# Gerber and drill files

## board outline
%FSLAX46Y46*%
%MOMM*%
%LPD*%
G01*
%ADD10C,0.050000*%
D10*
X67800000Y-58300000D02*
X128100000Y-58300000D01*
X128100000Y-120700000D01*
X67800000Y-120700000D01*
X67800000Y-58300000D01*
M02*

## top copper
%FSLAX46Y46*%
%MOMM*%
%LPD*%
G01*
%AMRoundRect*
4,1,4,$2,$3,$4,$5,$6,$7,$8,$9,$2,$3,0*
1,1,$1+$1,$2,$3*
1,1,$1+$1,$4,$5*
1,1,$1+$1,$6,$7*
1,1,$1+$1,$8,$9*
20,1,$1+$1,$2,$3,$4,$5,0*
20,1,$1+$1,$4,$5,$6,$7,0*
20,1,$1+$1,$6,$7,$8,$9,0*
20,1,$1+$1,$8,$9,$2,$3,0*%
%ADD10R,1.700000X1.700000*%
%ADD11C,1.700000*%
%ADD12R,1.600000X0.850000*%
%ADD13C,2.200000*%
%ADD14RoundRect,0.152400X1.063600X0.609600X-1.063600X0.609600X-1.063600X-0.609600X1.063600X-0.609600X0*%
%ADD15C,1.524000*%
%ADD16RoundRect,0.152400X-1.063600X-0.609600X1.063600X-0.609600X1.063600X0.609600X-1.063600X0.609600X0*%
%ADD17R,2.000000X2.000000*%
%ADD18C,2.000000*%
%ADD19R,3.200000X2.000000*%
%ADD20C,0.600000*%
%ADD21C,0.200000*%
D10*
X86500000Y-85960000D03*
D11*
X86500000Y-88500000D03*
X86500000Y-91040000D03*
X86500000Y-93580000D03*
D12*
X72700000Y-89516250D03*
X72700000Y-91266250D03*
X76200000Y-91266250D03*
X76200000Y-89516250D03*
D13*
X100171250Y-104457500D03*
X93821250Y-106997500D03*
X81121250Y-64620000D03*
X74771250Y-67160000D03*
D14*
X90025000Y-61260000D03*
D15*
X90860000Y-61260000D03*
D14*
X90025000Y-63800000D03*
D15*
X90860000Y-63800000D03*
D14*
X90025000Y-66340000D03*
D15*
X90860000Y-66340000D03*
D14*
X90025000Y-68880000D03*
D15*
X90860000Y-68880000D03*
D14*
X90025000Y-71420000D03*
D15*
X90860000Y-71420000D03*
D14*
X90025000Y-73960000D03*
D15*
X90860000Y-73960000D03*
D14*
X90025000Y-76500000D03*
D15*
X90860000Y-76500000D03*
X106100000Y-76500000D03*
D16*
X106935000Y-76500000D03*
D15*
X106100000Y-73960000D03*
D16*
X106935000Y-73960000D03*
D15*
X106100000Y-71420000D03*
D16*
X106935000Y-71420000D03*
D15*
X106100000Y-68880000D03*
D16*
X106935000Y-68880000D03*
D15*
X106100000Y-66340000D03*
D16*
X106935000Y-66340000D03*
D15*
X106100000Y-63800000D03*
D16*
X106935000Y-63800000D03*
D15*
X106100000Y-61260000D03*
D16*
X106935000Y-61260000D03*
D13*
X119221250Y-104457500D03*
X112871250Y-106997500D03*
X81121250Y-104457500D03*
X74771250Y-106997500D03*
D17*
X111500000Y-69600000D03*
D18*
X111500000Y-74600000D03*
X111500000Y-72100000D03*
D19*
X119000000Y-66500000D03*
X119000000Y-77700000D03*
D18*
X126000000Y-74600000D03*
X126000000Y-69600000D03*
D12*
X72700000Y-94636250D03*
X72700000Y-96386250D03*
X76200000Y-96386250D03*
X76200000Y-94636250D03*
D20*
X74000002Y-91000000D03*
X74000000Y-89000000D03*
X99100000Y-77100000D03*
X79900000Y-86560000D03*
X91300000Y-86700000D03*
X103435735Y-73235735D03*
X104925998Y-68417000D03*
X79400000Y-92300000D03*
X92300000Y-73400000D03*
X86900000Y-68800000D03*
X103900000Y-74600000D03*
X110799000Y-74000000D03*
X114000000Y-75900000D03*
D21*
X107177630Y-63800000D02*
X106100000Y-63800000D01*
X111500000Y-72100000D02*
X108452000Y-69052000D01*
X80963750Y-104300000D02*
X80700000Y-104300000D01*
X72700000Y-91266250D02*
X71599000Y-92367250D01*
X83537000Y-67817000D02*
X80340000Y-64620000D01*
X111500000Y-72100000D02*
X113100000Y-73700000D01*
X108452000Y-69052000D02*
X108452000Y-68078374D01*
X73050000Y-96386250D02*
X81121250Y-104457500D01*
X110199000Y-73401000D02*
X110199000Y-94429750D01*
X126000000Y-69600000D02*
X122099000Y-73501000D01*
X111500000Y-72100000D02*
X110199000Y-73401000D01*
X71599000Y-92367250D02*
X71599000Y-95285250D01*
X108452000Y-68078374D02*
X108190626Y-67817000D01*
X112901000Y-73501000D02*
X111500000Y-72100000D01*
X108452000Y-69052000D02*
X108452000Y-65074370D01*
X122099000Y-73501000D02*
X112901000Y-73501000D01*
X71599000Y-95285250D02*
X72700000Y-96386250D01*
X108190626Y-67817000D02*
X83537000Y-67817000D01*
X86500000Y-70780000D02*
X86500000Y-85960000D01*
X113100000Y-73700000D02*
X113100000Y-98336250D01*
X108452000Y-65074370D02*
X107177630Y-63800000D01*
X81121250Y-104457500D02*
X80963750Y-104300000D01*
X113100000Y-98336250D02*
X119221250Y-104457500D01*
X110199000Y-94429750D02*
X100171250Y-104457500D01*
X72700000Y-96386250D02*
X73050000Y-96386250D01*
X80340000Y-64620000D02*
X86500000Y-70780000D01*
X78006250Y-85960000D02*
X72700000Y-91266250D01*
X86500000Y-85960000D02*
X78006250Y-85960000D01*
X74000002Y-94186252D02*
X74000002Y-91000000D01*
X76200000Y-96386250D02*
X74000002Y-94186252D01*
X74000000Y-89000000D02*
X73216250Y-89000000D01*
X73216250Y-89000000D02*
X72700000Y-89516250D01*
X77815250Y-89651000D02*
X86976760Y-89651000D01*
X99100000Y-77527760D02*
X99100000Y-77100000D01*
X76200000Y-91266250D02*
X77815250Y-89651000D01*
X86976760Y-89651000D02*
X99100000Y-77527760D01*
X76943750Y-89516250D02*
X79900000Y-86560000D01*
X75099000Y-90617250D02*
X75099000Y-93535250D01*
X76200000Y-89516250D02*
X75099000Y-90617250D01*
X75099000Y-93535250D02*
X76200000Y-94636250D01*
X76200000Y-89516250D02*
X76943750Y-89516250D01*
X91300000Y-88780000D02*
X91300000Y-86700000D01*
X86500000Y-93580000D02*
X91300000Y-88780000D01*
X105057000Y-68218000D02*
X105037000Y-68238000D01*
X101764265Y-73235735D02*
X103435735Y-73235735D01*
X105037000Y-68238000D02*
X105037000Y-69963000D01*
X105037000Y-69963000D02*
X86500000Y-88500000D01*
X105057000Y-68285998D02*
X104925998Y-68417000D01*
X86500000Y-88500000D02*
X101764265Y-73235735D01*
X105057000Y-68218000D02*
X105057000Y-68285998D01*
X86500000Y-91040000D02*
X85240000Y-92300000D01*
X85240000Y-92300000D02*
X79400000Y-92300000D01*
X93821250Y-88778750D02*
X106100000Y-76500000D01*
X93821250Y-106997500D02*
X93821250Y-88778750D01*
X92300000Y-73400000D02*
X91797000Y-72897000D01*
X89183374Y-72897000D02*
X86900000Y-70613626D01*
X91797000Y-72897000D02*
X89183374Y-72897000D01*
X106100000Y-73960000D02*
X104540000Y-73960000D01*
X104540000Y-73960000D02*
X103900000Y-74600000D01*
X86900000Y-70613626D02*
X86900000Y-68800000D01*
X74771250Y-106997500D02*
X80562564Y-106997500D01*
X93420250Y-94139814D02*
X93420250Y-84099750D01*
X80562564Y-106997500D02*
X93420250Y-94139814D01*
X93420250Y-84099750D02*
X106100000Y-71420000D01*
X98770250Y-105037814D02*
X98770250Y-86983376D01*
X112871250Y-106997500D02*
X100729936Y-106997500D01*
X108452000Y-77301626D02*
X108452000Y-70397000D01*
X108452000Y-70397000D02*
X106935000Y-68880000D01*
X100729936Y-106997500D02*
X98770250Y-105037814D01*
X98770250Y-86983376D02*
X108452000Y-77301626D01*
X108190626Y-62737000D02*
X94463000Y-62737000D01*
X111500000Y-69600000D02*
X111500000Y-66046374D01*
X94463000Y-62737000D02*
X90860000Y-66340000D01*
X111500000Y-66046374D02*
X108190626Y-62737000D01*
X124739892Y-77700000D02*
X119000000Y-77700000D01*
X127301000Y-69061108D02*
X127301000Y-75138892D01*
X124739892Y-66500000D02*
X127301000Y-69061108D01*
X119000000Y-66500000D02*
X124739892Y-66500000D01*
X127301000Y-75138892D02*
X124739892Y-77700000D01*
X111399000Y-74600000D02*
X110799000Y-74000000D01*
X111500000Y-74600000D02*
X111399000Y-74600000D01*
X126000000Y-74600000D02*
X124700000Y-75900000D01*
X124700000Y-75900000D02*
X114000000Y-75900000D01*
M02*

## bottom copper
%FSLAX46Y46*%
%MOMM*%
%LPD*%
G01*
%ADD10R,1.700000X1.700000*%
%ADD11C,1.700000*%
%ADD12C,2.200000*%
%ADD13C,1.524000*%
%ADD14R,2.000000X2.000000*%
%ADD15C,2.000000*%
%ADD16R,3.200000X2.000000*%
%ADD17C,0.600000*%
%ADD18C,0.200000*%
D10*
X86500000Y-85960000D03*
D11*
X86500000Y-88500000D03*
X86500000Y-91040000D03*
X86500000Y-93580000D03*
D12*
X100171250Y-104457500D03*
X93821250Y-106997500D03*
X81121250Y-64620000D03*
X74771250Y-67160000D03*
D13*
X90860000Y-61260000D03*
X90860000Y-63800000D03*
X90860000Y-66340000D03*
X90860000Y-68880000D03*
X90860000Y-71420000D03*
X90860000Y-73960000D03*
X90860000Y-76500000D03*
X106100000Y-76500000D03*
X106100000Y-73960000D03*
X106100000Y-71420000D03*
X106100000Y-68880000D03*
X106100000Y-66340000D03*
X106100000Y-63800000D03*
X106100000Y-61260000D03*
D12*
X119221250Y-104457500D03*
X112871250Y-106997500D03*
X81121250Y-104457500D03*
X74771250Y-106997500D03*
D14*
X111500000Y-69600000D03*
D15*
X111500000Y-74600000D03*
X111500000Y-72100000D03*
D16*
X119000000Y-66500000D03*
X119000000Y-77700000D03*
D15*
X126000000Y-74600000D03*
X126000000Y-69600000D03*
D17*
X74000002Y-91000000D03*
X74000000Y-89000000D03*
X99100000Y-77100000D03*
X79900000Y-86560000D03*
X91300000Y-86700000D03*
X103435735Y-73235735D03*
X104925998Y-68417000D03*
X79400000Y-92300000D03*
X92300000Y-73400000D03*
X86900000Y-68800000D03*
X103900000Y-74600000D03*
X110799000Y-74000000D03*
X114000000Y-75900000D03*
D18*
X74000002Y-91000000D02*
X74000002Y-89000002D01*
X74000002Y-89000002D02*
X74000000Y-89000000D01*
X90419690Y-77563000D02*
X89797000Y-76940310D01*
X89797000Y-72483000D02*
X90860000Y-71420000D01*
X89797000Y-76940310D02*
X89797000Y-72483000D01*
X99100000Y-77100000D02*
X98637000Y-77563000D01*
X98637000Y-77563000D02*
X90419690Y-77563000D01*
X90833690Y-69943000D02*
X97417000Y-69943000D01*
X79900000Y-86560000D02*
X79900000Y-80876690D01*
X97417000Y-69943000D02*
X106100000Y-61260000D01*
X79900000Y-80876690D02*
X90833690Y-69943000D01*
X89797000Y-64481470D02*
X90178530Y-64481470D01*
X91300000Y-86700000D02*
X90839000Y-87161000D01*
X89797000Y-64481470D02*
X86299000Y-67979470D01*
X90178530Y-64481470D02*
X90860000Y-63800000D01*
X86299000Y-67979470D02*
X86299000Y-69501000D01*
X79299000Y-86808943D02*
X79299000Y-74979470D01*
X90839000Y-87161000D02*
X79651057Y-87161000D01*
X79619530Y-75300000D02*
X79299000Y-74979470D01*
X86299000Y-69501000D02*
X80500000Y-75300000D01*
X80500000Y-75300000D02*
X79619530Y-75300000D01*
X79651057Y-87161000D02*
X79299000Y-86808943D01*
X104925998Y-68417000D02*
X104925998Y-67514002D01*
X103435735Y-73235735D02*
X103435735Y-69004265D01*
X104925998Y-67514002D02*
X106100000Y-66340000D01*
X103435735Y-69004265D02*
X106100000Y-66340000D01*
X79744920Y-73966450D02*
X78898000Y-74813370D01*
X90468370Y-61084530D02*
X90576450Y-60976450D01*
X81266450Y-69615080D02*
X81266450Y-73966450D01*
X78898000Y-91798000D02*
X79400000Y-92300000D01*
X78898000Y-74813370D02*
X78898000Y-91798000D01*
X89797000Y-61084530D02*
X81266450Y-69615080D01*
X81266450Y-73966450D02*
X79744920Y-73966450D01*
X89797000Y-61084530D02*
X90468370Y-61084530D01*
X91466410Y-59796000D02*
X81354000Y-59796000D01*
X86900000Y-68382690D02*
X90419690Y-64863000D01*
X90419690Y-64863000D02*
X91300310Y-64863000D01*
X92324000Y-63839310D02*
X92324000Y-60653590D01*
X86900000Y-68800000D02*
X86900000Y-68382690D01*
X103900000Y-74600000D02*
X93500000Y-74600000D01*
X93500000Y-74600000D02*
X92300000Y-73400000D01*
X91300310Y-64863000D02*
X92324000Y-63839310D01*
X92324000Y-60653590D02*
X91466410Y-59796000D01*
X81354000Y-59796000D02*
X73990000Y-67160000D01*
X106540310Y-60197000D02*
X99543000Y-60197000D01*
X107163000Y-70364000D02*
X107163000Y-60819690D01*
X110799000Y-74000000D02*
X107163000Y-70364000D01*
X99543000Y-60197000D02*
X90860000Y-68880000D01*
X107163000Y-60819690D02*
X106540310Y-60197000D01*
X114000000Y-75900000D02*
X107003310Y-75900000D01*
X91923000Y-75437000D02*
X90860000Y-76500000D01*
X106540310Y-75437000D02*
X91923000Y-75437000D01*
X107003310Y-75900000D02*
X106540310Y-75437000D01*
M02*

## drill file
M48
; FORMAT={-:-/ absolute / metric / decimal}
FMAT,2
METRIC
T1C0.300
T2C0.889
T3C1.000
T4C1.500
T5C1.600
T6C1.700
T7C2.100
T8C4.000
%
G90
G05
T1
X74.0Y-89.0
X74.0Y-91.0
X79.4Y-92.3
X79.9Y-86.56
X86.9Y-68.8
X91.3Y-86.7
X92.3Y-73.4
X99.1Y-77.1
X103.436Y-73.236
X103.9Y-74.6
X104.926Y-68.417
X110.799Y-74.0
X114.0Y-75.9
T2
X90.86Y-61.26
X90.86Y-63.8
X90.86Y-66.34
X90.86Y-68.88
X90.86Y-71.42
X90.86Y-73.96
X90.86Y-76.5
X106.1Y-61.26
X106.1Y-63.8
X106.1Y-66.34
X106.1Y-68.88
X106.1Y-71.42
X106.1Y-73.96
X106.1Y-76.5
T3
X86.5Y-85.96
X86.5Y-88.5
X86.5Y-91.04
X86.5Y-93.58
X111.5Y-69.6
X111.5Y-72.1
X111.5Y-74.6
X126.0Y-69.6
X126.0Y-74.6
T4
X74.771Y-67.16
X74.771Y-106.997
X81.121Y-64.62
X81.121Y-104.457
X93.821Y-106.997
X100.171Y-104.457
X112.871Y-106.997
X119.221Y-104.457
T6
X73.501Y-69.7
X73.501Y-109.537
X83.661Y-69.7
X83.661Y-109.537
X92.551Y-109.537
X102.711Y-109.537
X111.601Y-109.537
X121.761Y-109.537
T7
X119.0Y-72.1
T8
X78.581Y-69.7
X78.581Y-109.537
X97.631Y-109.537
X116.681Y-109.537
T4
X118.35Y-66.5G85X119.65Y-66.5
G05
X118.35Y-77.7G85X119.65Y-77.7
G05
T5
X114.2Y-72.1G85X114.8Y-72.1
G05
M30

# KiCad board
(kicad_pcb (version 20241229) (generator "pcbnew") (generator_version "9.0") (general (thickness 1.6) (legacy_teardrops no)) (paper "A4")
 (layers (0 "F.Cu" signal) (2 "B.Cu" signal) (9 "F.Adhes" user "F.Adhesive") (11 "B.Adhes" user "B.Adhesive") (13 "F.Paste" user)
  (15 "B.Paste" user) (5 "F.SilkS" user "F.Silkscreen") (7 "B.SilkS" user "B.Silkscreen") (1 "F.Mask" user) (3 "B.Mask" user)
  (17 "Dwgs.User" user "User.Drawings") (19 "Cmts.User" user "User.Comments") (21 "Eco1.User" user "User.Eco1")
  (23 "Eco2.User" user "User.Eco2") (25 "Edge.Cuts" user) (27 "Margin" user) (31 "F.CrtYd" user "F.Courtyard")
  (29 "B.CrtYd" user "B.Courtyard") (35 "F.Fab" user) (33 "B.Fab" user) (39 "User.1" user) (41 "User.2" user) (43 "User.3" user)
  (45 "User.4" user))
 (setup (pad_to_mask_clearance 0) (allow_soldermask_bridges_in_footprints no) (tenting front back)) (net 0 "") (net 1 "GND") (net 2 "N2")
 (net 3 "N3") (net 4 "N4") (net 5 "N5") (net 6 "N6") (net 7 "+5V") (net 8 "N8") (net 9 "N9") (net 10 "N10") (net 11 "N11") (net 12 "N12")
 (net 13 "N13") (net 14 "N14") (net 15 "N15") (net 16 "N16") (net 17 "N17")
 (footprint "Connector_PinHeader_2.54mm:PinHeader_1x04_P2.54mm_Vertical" (layer "F.Cu") (at 86.5 85.96)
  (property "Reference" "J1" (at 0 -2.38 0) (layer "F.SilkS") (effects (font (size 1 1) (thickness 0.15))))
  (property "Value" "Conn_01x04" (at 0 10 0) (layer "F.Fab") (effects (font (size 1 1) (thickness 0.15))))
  (pad "1" thru_hole rect (at 0 0) (size 1.7 1.7) (drill 1) (layers "*.Cu" "*.Mask") (remove_unused_layers no) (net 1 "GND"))
  (pad "2" thru_hole circle (at 0 2.54) (size 1.7 1.7) (drill 1) (layers "*.Cu" "*.Mask") (remove_unused_layers no) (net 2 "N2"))
  (pad "3" thru_hole circle (at 0 5.08) (size 1.7 1.7) (drill 1) (layers "*.Cu" "*.Mask") (remove_unused_layers no) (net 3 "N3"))
  (pad "4" thru_hole circle (at 0 7.62) (size 1.7 1.7) (drill 1) (layers "*.Cu" "*.Mask") (remove_unused_layers no) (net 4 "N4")))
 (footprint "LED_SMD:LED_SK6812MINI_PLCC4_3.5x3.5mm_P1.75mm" (layer "F.Cu") (at 74.45 90.39125)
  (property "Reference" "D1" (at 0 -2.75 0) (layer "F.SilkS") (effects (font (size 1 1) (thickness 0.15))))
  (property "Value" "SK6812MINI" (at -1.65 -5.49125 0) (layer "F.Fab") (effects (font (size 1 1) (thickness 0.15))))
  (pad "1" smd rect (at -1.75 -0.875) (size 1.6 0.85) (layers "F.Cu" "F.Mask" "F.Paste") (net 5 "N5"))
  (pad "2" smd rect (at -1.75 0.875) (size 1.6 0.85) (layers "F.Cu" "F.Mask" "F.Paste") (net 1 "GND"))
  (pad "3" smd rect (at 1.75 0.875) (size 1.6 0.85) (layers "F.Cu" "F.Mask" "F.Paste") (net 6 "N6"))
  (pad "4" smd rect (at 1.75 -0.875) (size 1.6 0.85) (layers "F.Cu" "F.Mask" "F.Paste") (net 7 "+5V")))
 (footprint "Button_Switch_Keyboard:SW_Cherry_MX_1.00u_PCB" (layer "F.Cu") (at 100.17125 104.4575)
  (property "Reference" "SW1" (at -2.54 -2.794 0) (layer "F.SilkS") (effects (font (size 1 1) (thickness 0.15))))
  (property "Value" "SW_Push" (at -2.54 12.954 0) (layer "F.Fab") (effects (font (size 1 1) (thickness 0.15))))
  (pad "" np_thru_hole circle (at -7.62 5.08) (size 1.7 1.7) (drill 1.7) (layers "*.Cu" "*.Mask"))
  (pad "" np_thru_hole circle (at -2.54 5.08) (size 4 4) (drill 4) (layers "*.Cu" "*.Mask"))
  (pad "" np_thru_hole circle (at 2.54 5.08) (size 1.7 1.7) (drill 1.7) (layers "*.Cu" "*.Mask"))
  (pad "1" thru_hole circle (at 0 0) (size 2.2 2.2) (drill 1.5) (layers "*.Cu" "*.Mask") (remove_unused_layers no) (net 1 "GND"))
  (pad "2" thru_hole circle (at -6.35 2.54) (size 2.2 2.2) (drill 1.5) (layers "*.Cu" "*.Mask") (remove_unused_layers no) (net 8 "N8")))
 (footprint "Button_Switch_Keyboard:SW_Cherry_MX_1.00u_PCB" (layer "F.Cu") (at 81.12125 64.62)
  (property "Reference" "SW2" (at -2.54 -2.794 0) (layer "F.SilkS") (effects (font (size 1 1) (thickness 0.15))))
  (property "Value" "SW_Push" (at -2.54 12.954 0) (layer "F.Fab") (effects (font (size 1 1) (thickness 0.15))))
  (pad "" np_thru_hole circle (at -7.62 5.08) (size 1.7 1.7) (drill 1.7) (layers "*.Cu" "*.Mask"))
  (pad "" np_thru_hole circle (at -2.54 5.08) (size 4 4) (drill 4) (layers "*.Cu" "*.Mask"))
  (pad "" np_thru_hole circle (at 2.54 5.08) (size 1.7 1.7) (drill 1.7) (layers "*.Cu" "*.Mask"))
  (pad "1" thru_hole circle (at 0 0) (size 2.2 2.2) (drill 1.5) (layers "*.Cu" "*.Mask") (remove_unused_layers no) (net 1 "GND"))
  (pad "2" thru_hole circle (at -6.35 2.54) (size 2.2 2.2) (drill 1.5) (layers "*.Cu" "*.Mask") (remove_unused_layers no) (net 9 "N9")))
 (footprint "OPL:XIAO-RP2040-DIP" (layer "F.Cu") (at 98.48 68.88)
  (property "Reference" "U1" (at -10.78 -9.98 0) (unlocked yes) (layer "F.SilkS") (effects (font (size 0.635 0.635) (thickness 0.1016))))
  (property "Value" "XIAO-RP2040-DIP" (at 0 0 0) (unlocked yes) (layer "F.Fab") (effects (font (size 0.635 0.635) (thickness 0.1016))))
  (pad "1" smd roundrect (at -8.455 -7.62 180) (size 2.432 1.524) (layers "F.Cu" "F.Mask") (roundrect_rratio 0.1) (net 3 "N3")
   (thermal_bridge_angle 45))
  (pad "1" thru_hole circle (at -7.62 -7.62 180) (size 1.524 1.524) (drill 0.889) (layers "*.Cu" "*.Mask") (remove_unused_layers no)
   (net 3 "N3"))
  (pad "2" smd roundrect (at -8.455 -5.08 180) (size 2.432 1.524) (layers "F.Cu" "F.Mask") (roundrect_rratio 0.1) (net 4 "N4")
   (thermal_bridge_angle 45))
  (pad "2" thru_hole circle (at -7.62 -5.08 180) (size 1.524 1.524) (drill 0.889) (layers "*.Cu" "*.Mask") (remove_unused_layers no)
   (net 4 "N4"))
  (pad "3" smd roundrect (at -8.455 -2.54 180) (size 2.432 1.524) (layers "F.Cu" "F.Mask") (roundrect_rratio 0.1) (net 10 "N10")
   (thermal_bridge_angle 45))
  (pad "3" thru_hole circle (at -7.62 -2.54 180) (size 1.524 1.524) (drill 0.889) (layers "*.Cu" "*.Mask") (remove_unused_layers no)
   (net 10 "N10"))
  (pad "4" smd roundrect (at -8.455 0 180) (size 2.432 1.524) (layers "F.Cu" "F.Mask") (roundrect_rratio 0.1) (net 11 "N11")
   (thermal_bridge_angle 45))
  (pad "4" thru_hole circle (at -7.62 0 180) (size 1.524 1.524) (drill 0.889) (layers "*.Cu" "*.Mask") (remove_unused_layers no)
   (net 11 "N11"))
  (pad "5" smd roundrect (at -8.455 2.54 180) (size 2.432 1.524) (layers "F.Cu" "F.Mask") (roundrect_rratio 0.1) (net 6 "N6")
   (thermal_bridge_angle 45))
  (pad "5" thru_hole circle (at -7.62 2.54 180) (size 1.524 1.524) (drill 0.889) (layers "*.Cu" "*.Mask") (remove_unused_layers no)
   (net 6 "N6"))
  (pad "6" smd roundrect (at -8.455 5.08 180) (size 2.432 1.524) (layers "F.Cu" "F.Mask") (roundrect_rratio 0.1) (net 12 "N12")
   (thermal_bridge_angle 45))
  (pad "6" thru_hole circle (at -7.62 5.08 180) (size 1.524 1.524) (drill 0.889) (layers "*.Cu" "*.Mask") (remove_unused_layers no)
   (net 12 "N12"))
  (pad "7" smd roundrect (at -8.455 7.62 180) (size 2.432 1.524) (layers "F.Cu" "F.Mask") (roundrect_rratio 0.1) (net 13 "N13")
   (thermal_bridge_angle 45))
  (pad "7" thru_hole circle (at -7.62 7.62 180) (size 1.524 1.524) (drill 0.889) (layers "*.Cu" "*.Mask") (remove_unused_layers no)
   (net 13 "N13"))
  (pad "8" thru_hole circle (at 7.62 7.62) (size 1.524 1.524) (drill 0.889) (layers "*.Cu" "*.Mask") (remove_unused_layers no) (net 8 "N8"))
  (pad "8" smd roundrect (at 8.455 7.62) (size 2.432 1.524) (layers "F.Cu" "F.Mask") (roundrect_rratio 0.1) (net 8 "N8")
   (thermal_bridge_angle 45))
  (pad "9" thru_hole circle (at 7.62 5.08) (size 1.524 1.524) (drill 0.889) (layers "*.Cu" "*.Mask") (remove_unused_layers no) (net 9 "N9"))
  (pad "9" smd roundrect (at 8.455 5.08) (size 2.432 1.524) (layers "F.Cu" "F.Mask") (roundrect_rratio 0.1) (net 9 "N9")
   (thermal_bridge_angle 45))
  (pad "10" thru_hole circle (at 7.62 2.54) (size 1.524 1.524) (drill 0.889) (layers "*.Cu" "*.Mask") (remove_unused_layers no)
   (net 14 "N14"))
  (pad "10" smd roundrect (at 8.455 2.54) (size 2.432 1.524) (layers "F.Cu" "F.Mask") (roundrect_rratio 0.1) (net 14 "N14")
   (thermal_bridge_angle 45))
  (pad "11" thru_hole circle (at 7.62 0) (size 1.524 1.524) (drill 0.889) (layers "*.Cu" "*.Mask") (remove_unused_layers no) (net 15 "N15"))
  (pad "11" smd roundrect (at 8.455 0) (size 2.432 1.524) (layers "F.Cu" "F.Mask") (roundrect_rratio 0.1) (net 15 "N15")
   (thermal_bridge_angle 45))
  (pad "12" thru_hole circle (at 7.62 -2.54) (size 1.524 1.524) (drill 0.889) (layers "*.Cu" "*.Mask") (remove_unused_layers no)
   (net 2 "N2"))
  (pad "12" smd roundrect (at 8.455 -2.54) (size 2.432 1.524) (layers "F.Cu" "F.Mask") (roundrect_rratio 0.1) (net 2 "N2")
   (thermal_bridge_angle 45))
  (pad "13" thru_hole circle (at 7.62 -5.08) (size 1.524 1.524) (drill 0.889) (layers "*.Cu" "*.Mask") (remove_unused_layers no)
   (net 1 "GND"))
  (pad "13" smd roundrect (at 8.455 -5.08) (size 2.432 1.524) (layers "F.Cu" "F.Mask") (roundrect_rratio 0.1) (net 1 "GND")
   (thermal_bridge_angle 45))
  (pad "14" thru_hole circle (at 7.62 -7.62) (size 1.524 1.524) (drill 0.889) (layers "*.Cu" "*.Mask") (remove_unused_layers no)
   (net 7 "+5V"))
  (pad "14" smd roundrect (at 8.455 -7.62) (size 2.432 1.524) (layers "F.Cu" "F.Mask") (roundrect_rratio 0.1) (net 7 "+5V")
   (thermal_bridge_angle 45)))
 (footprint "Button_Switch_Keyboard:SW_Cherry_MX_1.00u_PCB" (layer "F.Cu") (at 119.22125 104.4575)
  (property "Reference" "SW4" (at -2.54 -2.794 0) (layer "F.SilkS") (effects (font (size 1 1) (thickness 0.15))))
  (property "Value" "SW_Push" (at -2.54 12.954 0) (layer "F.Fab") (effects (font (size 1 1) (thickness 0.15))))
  (pad "" np_thru_hole circle (at -7.62 5.08) (size 1.7 1.7) (drill 1.7) (layers "*.Cu" "*.Mask"))
  (pad "" np_thru_hole circle (at -2.54 5.08) (size 4 4) (drill 4) (layers "*.Cu" "*.Mask"))
  (pad "" np_thru_hole circle (at 2.54 5.08) (size 1.7 1.7) (drill 1.7) (layers "*.Cu" "*.Mask"))
  (pad "1" thru_hole circle (at 0 0) (size 2.2 2.2) (drill 1.5) (layers "*.Cu" "*.Mask") (remove_unused_layers no) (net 1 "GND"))
  (pad "2" thru_hole circle (at -6.35 2.54) (size 2.2 2.2) (drill 1.5) (layers "*.Cu" "*.Mask") (remove_unused_layers no) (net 15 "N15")))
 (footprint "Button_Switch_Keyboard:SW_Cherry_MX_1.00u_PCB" (layer "F.Cu") (at 81.12125 104.4575)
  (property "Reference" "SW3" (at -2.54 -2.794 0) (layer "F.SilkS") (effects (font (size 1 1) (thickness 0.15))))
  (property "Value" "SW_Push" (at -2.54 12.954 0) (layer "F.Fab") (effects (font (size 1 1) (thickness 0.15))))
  (pad "" np_thru_hole circle (at -7.62 5.08) (size 1.7 1.7) (drill 1.7) (layers "*.Cu" "*.Mask"))
  (pad "" np_thru_hole circle (at -2.54 5.08) (size 4 4) (drill 4) (layers "*.Cu" "*.Mask"))
  (pad "" np_thru_hole circle (at 2.54 5.08) (size 1.7 1.7) (drill 1.7) (layers "*.Cu" "*.Mask"))
  (pad "1" thru_hole circle (at 0 0) (size 2.2 2.2) (drill 1.5) (layers "*.Cu" "*.Mask") (remove_unused_layers no) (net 1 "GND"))
  (pad "2" thru_hole circle (at -6.35 2.54) (size 2.2 2.2) (drill 1.5) (layers "*.Cu" "*.Mask") (remove_unused_layers no) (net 14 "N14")))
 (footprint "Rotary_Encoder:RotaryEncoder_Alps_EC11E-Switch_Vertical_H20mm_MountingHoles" (layer "F.Cu") (at 111.5 69.6)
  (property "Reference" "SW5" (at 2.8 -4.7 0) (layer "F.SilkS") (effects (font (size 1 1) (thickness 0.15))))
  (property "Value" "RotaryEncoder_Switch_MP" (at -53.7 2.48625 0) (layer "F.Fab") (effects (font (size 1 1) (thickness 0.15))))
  (pad "" np_thru_hole oval (at 3 2.5) (size 2.2 1.6) (drill oval 2.2 1.6) (layers "*.Mask"))
  (pad "" np_thru_hole circle (at 7.5 2.5) (size 2.1 2.1) (drill 2.1) (layers "*.Mask"))
  (pad "A" thru_hole rect (at 0 0) (size 2 2) (drill 1) (layers "*.Cu" "*.Mask") (remove_unused_layers no) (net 10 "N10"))
  (pad "B" thru_hole circle (at 0 5) (size 2 2) (drill 1) (layers "*.Cu" "*.Mask") (remove_unused_layers no) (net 11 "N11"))
  (pad "C" thru_hole circle (at 0 2.5) (size 2 2) (drill 1) (layers "*.Cu" "*.Mask") (remove_unused_layers no) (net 1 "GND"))
  (pad "MP" thru_hole rect (at 7.5 -3.1) (size 3.2 2) (drill oval 2.8 1.5) (layers "*.Cu" "*.Mask") (remove_unused_layers no) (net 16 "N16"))
  (pad "MP" thru_hole rect (at 7.5 8.1) (size 3.2 2) (drill oval 2.8 1.5) (layers "*.Cu" "*.Mask") (remove_unused_layers no) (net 16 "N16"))
  (pad "S1" thru_hole circle (at 14.5 5) (size 2 2) (drill 1) (layers "*.Cu" "*.Mask") (remove_unused_layers no) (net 13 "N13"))
  (pad "S2" thru_hole circle (at 14.5 0) (size 2 2) (drill 1) (layers "*.Cu" "*.Mask") (remove_unused_layers no) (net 1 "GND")))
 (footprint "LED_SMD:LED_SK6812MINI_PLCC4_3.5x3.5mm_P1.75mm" (layer "F.Cu") (at 74.45 95.51125)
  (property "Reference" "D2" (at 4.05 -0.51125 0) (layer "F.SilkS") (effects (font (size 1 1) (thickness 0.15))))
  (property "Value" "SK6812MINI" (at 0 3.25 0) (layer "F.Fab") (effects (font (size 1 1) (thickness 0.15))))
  (pad "1" smd rect (at -1.75 -0.875) (size 1.6 0.85) (layers "F.Cu" "F.Mask" "F.Paste") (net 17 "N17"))
  (pad "2" smd rect (at -1.75 0.875) (size 1.6 0.85) (layers "F.Cu" "F.Mask" "F.Paste") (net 1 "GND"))
  (pad "3" smd rect (at 1.75 0.875) (size 1.6 0.85) (layers "F.Cu" "F.Mask" "F.Paste") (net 5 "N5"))
  (pad "4" smd rect (at 1.75 -0.875) (size 1.6 0.85) (layers "F.Cu" "F.Mask" "F.Paste") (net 7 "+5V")))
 (gr_rect (start 67.8 58.3) (end 128.1 120.7) (stroke (width 0.05) (type default)) (fill no) (layer "Edge.Cuts"))
 (segment (start 107.17763 63.8) (end 106.1 63.8) (width 0.2) (layer "F.Cu") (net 1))
 (segment (start 111.5 72.1) (end 108.452 69.052) (width 0.2) (layer "F.Cu") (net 1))
 (segment (start 80.96375 104.3) (end 80.7 104.3) (width 0.2) (layer "F.Cu") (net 1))
 (segment (start 72.7 91.26625) (end 71.599 92.36725) (width 0.2) (layer "F.Cu") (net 1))
 (segment (start 83.537 67.817) (end 80.34 64.62) (width 0.2) (layer "F.Cu") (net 1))
 (segment (start 111.5 72.1) (end 113.1 73.7) (width 0.2) (layer "F.Cu") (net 1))
 (segment (start 108.452 69.052) (end 108.452 68.078374) (width 0.2) (layer "F.Cu") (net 1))
 (segment (start 73.05 96.38625) (end 81.12125 104.4575) (width 0.2) (layer "F.Cu") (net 1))
 (segment (start 110.199 73.401) (end 110.199 94.42975) (width 0.2) (layer "F.Cu") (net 1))
 (segment (start 126 69.6) (end 122.099 73.501) (width 0.2) (layer "F.Cu") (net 1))
 (segment (start 111.5 72.1) (end 110.199 73.401) (width 0.2) (layer "F.Cu") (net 1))
 (segment (start 71.599 92.36725) (end 71.599 95.28525) (width 0.2) (layer "F.Cu") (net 1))
 (segment (start 108.452 68.078374) (end 108.190626 67.817) (width 0.2) (layer "F.Cu") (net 1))
 (segment (start 112.901 73.501) (end 111.5 72.1) (width 0.2) (layer "F.Cu") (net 1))
 (segment (start 108.452 69.052) (end 108.452 65.07437) (width 0.2) (layer "F.Cu") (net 1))
 (segment (start 122.099 73.501) (end 112.901 73.501) (width 0.2) (layer "F.Cu") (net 1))
 (segment (start 71.599 95.28525) (end 72.7 96.38625) (width 0.2) (layer "F.Cu") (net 1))
 (segment (start 108.190626 67.817) (end 83.537 67.817) (width 0.2) (layer "F.Cu") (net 1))
 (segment (start 86.5 70.78) (end 86.5 85.96) (width 0.2) (layer "F.Cu") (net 1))
 (segment (start 113.1 73.7) (end 113.1 98.33625) (width 0.2) (layer "F.Cu") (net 1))
 (segment (start 108.452 65.07437) (end 107.17763 63.8) (width 0.2) (layer "F.Cu") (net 1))
 (segment (start 81.12125 104.4575) (end 80.96375 104.3) (width 0.2) (layer "F.Cu") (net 1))
 (segment (start 113.1 98.33625) (end 119.22125 104.4575) (width 0.2) (layer "F.Cu") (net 1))
 (segment (start 110.199 94.42975) (end 100.17125 104.4575) (width 0.2) (layer "F.Cu") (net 1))
 (segment (start 72.7 96.38625) (end 73.05 96.38625) (width 0.2) (layer "F.Cu") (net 1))
 (segment (start 80.34 64.62) (end 86.5 70.78) (width 0.2) (layer "F.Cu") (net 1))
 (segment (start 78.00625 85.96) (end 72.7 91.26625) (width 0.2) (layer "F.Cu") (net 1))
 (segment (start 86.5 85.96) (end 78.00625 85.96) (width 0.2) (layer "F.Cu") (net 1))
 (segment (start 74.000002 94.186252) (end 74.000002 91) (width 0.2) (layer "F.Cu") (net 5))
 (segment (start 76.2 96.38625) (end 74.000002 94.186252) (width 0.2) (layer "F.Cu") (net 5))
 (segment (start 74 89) (end 73.21625 89) (width 0.2) (layer "F.Cu") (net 5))
 (segment (start 73.21625 89) (end 72.7 89.51625) (width 0.2) (layer "F.Cu") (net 5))
 (via (at 74.000002 91) (size 0.6) (drill 0.3) (layers "F.Cu" "B.Cu") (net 5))
 (via (at 74 89) (size 0.6) (drill 0.3) (layers "F.Cu" "B.Cu") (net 5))
 (segment (start 74.000002 91) (end 74.000002 89.000002) (width 0.2) (layer "B.Cu") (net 5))
 (segment (start 74.000002 89.000002) (end 74 89) (width 0.2) (layer "B.Cu") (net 5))
 (segment (start 77.81525 89.651) (end 86.97676 89.651) (width 0.2) (layer "F.Cu") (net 6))
 (segment (start 99.1 77.52776) (end 99.1 77.1) (width 0.2) (layer "F.Cu") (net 6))
 (segment (start 76.2 91.26625) (end 77.81525 89.651) (width 0.2) (layer "F.Cu") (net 6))
 (segment (start 86.97676 89.651) (end 99.1 77.52776) (width 0.2) (layer "F.Cu") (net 6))
 (via (at 99.1 77.1) (size 0.6) (drill 0.3) (layers "F.Cu" "B.Cu") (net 6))
 (segment (start 90.41969 77.563) (end 89.797 76.94031) (width 0.2) (layer "B.Cu") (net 6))
 (segment (start 89.797 72.483) (end 90.86 71.42) (width 0.2) (layer "B.Cu") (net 6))
 (segment (start 89.797 76.94031) (end 89.797 72.483) (width 0.2) (layer "B.Cu") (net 6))
 (segment (start 99.1 77.1) (end 98.637 77.563) (width 0.2) (layer "B.Cu") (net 6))
 (segment (start 98.637 77.563) (end 90.41969 77.563) (width 0.2) (layer "B.Cu") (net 6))
 (segment (start 76.94375 89.51625) (end 79.9 86.56) (width 0.2) (layer "F.Cu") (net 7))
 (segment (start 75.099 90.61725) (end 75.099 93.53525) (width 0.2) (layer "F.Cu") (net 7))
 (segment (start 76.2 89.51625) (end 75.099 90.61725) (width 0.2) (layer "F.Cu") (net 7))
 (segment (start 75.099 93.53525) (end 76.2 94.63625) (width 0.2) (layer "F.Cu") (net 7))
 (segment (start 76.2 89.51625) (end 76.94375 89.51625) (width 0.2) (layer "F.Cu") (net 7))
 (via (at 79.9 86.56) (size 0.6) (drill 0.3) (layers "F.Cu" "B.Cu") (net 7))
 (segment (start 90.83369 69.943) (end 97.417 69.943) (width 0.2) (layer "B.Cu") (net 7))
 (segment (start 79.9 86.56) (end 79.9 80.87669) (width 0.2) (layer "B.Cu") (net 7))
 (segment (start 97.417 69.943) (end 106.1 61.26) (width 0.2) (layer "B.Cu") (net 7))
 (segment (start 79.9 80.87669) (end 90.83369 69.943) (width 0.2) (layer "B.Cu") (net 7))
 (segment (start 91.3 88.78) (end 91.3 86.7) (width 0.2) (layer "F.Cu") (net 4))
 (segment (start 86.5 93.58) (end 91.3 88.78) (width 0.2) (layer "F.Cu") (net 4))
 (via (at 91.3 86.7) (size 0.6) (drill 0.3) (layers "F.Cu" "B.Cu") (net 4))
 (segment (start 89.797 64.48147) (end 90.17853 64.48147) (width 0.2) (layer "B.Cu") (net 4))
 (segment (start 91.3 86.7) (end 90.839 87.161) (width 0.2) (layer "B.Cu") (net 4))
 (segment (start 89.797 64.48147) (end 86.299 67.97947) (width 0.2) (layer "B.Cu") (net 4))
 (segment (start 90.17853 64.48147) (end 90.86 63.8) (width 0.2) (layer "B.Cu") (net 4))
 (segment (start 86.299 67.97947) (end 86.299 69.501) (width 0.2) (layer "B.Cu") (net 4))
 (segment (start 79.299 86.808943) (end 79.299 74.97947) (width 0.2) (layer "B.Cu") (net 4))
 (segment (start 90.839 87.161) (end 79.651057 87.161) (width 0.2) (layer "B.Cu") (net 4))
 (segment (start 79.61953 75.3) (end 79.299 74.97947) (width 0.2) (layer "B.Cu") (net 4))
 (segment (start 86.299 69.501) (end 80.5 75.3) (width 0.2) (layer "B.Cu") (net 4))
 (segment (start 80.5 75.3) (end 79.61953 75.3) (width 0.2) (layer "B.Cu") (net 4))
 (segment (start 79.651057 87.161) (end 79.299 86.808943) (width 0.2) (layer "B.Cu") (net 4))
 (segment (start 105.057 68.218) (end 105.037 68.238) (width 0.2) (layer "F.Cu") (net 2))
 (segment (start 101.764265 73.235735) (end 103.435735 73.235735) (width 0.2) (layer "F.Cu") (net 2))
 (segment (start 105.037 68.238) (end 105.037 69.963) (width 0.2) (layer "F.Cu") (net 2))
 (segment (start 105.037 69.963) (end 86.5 88.5) (width 0.2) (layer "F.Cu") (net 2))
 (segment (start 105.057 68.285998) (end 104.925998 68.417) (width 0.2) (layer "F.Cu") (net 2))
 (segment (start 86.5 88.5) (end 101.764265 73.235735) (width 0.2) (layer "F.Cu") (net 2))
 (segment (start 105.057 68.218) (end 105.057 68.285998) (width 0.2) (layer "F.Cu") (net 2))
 (via (at 103.435735 73.235735) (size 0.6) (drill 0.3) (layers "F.Cu" "B.Cu") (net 2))
 (via (at 104.925998 68.417) (size 0.6) (drill 0.3) (layers "F.Cu" "B.Cu") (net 2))
 (segment (start 104.925998 68.417) (end 104.925998 67.514002) (width 0.2) (layer "B.Cu") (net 2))
 (segment (start 103.435735 73.235735) (end 103.435735 69.004265) (width 0.2) (layer "B.Cu") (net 2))
 (segment (start 104.925998 67.514002) (end 106.1 66.34) (width 0.2) (layer "B.Cu") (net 2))
 (segment (start 103.435735 69.004265) (end 106.1 66.34) (width 0.2) (layer "B.Cu") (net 2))
 (segment (start 86.5 91.04) (end 85.24 92.3) (width 0.2) (layer "F.Cu") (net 3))
 (segment (start 85.24 92.3) (end 79.4 92.3) (width 0.2) (layer "F.Cu") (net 3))
 (via (at 79.4 92.3) (size 0.6) (drill 0.3) (layers "F.Cu" "B.Cu") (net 3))
 (segment (start 79.74492 73.96645) (end 78.898 74.81337) (width 0.2) (layer "B.Cu") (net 3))
 (segment (start 90.46837 61.08453) (end 90.57645 60.97645) (width 0.2) (layer "B.Cu") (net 3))
 (segment (start 81.26645 69.61508) (end 81.26645 73.96645) (width 0.2) (layer "B.Cu") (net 3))
 (segment (start 78.898 91.798) (end 79.4 92.3) (width 0.2) (layer "B.Cu") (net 3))
 (segment (start 78.898 74.81337) (end 78.898 91.798) (width 0.2) (layer "B.Cu") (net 3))
 (segment (start 89.797 61.08453) (end 81.26645 69.61508) (width 0.2) (layer "B.Cu") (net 3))
 (segment (start 81.26645 73.96645) (end 79.74492 73.96645) (width 0.2) (layer "B.Cu") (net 3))
 (segment (start 89.797 61.08453) (end 90.46837 61.08453) (width 0.2) (layer "B.Cu") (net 3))
 (segment (start 93.82125 88.77875) (end 106.1 76.5) (width 0.2) (layer "F.Cu") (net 8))
 (segment (start 93.82125 106.9975) (end 93.82125 88.77875) (width 0.2) (layer "F.Cu") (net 8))
 (segment (start 92.3 73.4) (end 91.797 72.897) (width 0.2) (layer "F.Cu") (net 9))
 (segment (start 89.183374 72.897) (end 86.9 70.613626) (width 0.2) (layer "F.Cu") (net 9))
 (segment (start 91.797 72.897) (end 89.183374 72.897) (width 0.2) (layer "F.Cu") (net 9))
 (segment (start 106.1 73.96) (end 104.54 73.96) (width 0.2) (layer "F.Cu") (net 9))
 (segment (start 104.54 73.96) (end 103.9 74.6) (width 0.2) (layer "F.Cu") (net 9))
 (segment (start 86.9 70.613626) (end 86.9 68.8) (width 0.2) (layer "F.Cu") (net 9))
 (via (at 92.3 73.4) (size 0.6) (drill 0.3) (layers "F.Cu" "B.Cu") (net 9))
 (via (at 86.9 68.8) (size 0.6) (drill 0.3) (layers "F.Cu" "B.Cu") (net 9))
 (via (at 103.9 74.6) (size 0.6) (drill 0.3) (layers "F.Cu" "B.Cu") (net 9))
 (segment (start 91.46641 59.796) (end 81.354 59.796) (width 0.2) (layer "B.Cu") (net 9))
 (segment (start 86.9 68.38269) (end 90.41969 64.863) (width 0.2) (layer "B.Cu") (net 9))
 (segment (start 90.41969 64.863) (end 91.30031 64.863) (width 0.2) (layer "B.Cu") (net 9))
 (segment (start 92.324 63.83931) (end 92.324 60.65359) (width 0.2) (layer "B.Cu") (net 9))
 (segment (start 86.9 68.8) (end 86.9 68.38269) (width 0.2) (layer "B.Cu") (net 9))
 (segment (start 103.9 74.6) (end 93.5 74.6) (width 0.2) (layer "B.Cu") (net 9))
 (segment (start 93.5 74.6) (end 92.3 73.4) (width 0.2) (layer "B.Cu") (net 9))
 (segment (start 91.30031 64.863) (end 92.324 63.83931) (width 0.2) (layer "B.Cu") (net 9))
 (segment (start 92.324 60.65359) (end 91.46641 59.796) (width 0.2) (layer "B.Cu") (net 9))
 (segment (start 81.354 59.796) (end 73.99 67.16) (width 0.2) (layer "B.Cu") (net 9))
 (segment (start 74.77125 106.9975) (end 80.562564 106.9975) (width 0.2) (layer "F.Cu") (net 14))
 (segment (start 93.42025 94.139814) (end 93.42025 84.09975) (width 0.2) (layer "F.Cu") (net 14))
 (segment (start 80.562564 106.9975) (end 93.42025 94.139814) (width 0.2) (layer "F.Cu") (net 14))
 (segment (start 93.42025 84.09975) (end 106.1 71.42) (width 0.2) (layer "F.Cu") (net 14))
 (segment (start 98.77025 105.037814) (end 98.77025 86.983376) (width 0.2) (layer "F.Cu") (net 15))
 (segment (start 112.87125 106.9975) (end 100.729936 106.9975) (width 0.2) (layer "F.Cu") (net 15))
 (segment (start 108.452 77.301626) (end 108.452 70.397) (width 0.2) (layer "F.Cu") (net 15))
 (segment (start 108.452 70.397) (end 106.935 68.88) (width 0.2) (layer "F.Cu") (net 15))
 (segment (start 100.729936 106.9975) (end 98.77025 105.037814) (width 0.2) (layer "F.Cu") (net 15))
 (segment (start 98.77025 86.983376) (end 108.452 77.301626) (width 0.2) (layer "F.Cu") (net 15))
 (segment (start 108.190626 62.737) (end 94.463 62.737) (width 0.2) (layer "F.Cu") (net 10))
 (segment (start 111.5 69.6) (end 111.5 66.046374) (width 0.2) (layer "F.Cu") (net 10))
 (segment (start 94.463 62.737) (end 90.86 66.34) (width 0.2) (layer "F.Cu") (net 10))
 (segment (start 111.5 66.046374) (end 108.190626 62.737) (width 0.2) (layer "F.Cu") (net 10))
 (segment (start 124.739892 77.7) (end 119 77.7) (width 0.2) (layer "F.Cu") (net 16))
 (segment (start 127.301 69.061108) (end 127.301 75.138892) (width 0.2) (layer "F.Cu") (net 16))
 (segment (start 124.739892 66.5) (end 127.301 69.061108) (width 0.2) (layer "F.Cu") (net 16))
 (segment (start 119 66.5) (end 124.739892 66.5) (width 0.2) (layer "F.Cu") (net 16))
 (segment (start 127.301 75.138892) (end 124.739892 77.7) (width 0.2) (layer "F.Cu") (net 16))
 (segment (start 111.399 74.6) (end 110.799 74) (width 0.2) (layer "F.Cu") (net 11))
 (segment (start 111.5 74.6) (end 111.399 74.6) (width 0.2) (layer "F.Cu") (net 11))
 (via (at 110.799 74) (size 0.6) (drill 0.3) (layers "F.Cu" "B.Cu") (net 11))
 (segment (start 106.54031 60.197) (end 99.543 60.197) (width 0.2) (layer "B.Cu") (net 11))
 (segment (start 107.163 70.364) (end 107.163 60.81969) (width 0.2) (layer "B.Cu") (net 11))
 (segment (start 110.799 74) (end 107.163 70.364) (width 0.2) (layer "B.Cu") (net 11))
 (segment (start 99.543 60.197) (end 90.86 68.88) (width 0.2) (layer "B.Cu") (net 11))
 (segment (start 107.163 60.81969) (end 106.54031 60.197) (width 0.2) (layer "B.Cu") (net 11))
 (segment (start 126 74.6) (end 124.7 75.9) (width 0.2) (layer "F.Cu") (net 13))
 (segment (start 124.7 75.9) (end 114 75.9) (width 0.2) (layer "F.Cu") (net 13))
 (via (at 114 75.9) (size 0.6) (drill 0.3) (layers "F.Cu" "B.Cu") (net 13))
 (segment (start 114 75.9) (end 107.00331 75.9) (width 0.2) (layer "B.Cu") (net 13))
 (segment (start 91.923 75.437) (end 90.86 76.5) (width 0.2) (layer "B.Cu") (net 13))
 (segment (start 106.54031 75.437) (end 91.923 75.437) (width 0.2) (layer "B.Cu") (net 13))
 (segment (start 107.00331 75.9) (end 106.54031 75.437) (width 0.2) (layer "B.Cu") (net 13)))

